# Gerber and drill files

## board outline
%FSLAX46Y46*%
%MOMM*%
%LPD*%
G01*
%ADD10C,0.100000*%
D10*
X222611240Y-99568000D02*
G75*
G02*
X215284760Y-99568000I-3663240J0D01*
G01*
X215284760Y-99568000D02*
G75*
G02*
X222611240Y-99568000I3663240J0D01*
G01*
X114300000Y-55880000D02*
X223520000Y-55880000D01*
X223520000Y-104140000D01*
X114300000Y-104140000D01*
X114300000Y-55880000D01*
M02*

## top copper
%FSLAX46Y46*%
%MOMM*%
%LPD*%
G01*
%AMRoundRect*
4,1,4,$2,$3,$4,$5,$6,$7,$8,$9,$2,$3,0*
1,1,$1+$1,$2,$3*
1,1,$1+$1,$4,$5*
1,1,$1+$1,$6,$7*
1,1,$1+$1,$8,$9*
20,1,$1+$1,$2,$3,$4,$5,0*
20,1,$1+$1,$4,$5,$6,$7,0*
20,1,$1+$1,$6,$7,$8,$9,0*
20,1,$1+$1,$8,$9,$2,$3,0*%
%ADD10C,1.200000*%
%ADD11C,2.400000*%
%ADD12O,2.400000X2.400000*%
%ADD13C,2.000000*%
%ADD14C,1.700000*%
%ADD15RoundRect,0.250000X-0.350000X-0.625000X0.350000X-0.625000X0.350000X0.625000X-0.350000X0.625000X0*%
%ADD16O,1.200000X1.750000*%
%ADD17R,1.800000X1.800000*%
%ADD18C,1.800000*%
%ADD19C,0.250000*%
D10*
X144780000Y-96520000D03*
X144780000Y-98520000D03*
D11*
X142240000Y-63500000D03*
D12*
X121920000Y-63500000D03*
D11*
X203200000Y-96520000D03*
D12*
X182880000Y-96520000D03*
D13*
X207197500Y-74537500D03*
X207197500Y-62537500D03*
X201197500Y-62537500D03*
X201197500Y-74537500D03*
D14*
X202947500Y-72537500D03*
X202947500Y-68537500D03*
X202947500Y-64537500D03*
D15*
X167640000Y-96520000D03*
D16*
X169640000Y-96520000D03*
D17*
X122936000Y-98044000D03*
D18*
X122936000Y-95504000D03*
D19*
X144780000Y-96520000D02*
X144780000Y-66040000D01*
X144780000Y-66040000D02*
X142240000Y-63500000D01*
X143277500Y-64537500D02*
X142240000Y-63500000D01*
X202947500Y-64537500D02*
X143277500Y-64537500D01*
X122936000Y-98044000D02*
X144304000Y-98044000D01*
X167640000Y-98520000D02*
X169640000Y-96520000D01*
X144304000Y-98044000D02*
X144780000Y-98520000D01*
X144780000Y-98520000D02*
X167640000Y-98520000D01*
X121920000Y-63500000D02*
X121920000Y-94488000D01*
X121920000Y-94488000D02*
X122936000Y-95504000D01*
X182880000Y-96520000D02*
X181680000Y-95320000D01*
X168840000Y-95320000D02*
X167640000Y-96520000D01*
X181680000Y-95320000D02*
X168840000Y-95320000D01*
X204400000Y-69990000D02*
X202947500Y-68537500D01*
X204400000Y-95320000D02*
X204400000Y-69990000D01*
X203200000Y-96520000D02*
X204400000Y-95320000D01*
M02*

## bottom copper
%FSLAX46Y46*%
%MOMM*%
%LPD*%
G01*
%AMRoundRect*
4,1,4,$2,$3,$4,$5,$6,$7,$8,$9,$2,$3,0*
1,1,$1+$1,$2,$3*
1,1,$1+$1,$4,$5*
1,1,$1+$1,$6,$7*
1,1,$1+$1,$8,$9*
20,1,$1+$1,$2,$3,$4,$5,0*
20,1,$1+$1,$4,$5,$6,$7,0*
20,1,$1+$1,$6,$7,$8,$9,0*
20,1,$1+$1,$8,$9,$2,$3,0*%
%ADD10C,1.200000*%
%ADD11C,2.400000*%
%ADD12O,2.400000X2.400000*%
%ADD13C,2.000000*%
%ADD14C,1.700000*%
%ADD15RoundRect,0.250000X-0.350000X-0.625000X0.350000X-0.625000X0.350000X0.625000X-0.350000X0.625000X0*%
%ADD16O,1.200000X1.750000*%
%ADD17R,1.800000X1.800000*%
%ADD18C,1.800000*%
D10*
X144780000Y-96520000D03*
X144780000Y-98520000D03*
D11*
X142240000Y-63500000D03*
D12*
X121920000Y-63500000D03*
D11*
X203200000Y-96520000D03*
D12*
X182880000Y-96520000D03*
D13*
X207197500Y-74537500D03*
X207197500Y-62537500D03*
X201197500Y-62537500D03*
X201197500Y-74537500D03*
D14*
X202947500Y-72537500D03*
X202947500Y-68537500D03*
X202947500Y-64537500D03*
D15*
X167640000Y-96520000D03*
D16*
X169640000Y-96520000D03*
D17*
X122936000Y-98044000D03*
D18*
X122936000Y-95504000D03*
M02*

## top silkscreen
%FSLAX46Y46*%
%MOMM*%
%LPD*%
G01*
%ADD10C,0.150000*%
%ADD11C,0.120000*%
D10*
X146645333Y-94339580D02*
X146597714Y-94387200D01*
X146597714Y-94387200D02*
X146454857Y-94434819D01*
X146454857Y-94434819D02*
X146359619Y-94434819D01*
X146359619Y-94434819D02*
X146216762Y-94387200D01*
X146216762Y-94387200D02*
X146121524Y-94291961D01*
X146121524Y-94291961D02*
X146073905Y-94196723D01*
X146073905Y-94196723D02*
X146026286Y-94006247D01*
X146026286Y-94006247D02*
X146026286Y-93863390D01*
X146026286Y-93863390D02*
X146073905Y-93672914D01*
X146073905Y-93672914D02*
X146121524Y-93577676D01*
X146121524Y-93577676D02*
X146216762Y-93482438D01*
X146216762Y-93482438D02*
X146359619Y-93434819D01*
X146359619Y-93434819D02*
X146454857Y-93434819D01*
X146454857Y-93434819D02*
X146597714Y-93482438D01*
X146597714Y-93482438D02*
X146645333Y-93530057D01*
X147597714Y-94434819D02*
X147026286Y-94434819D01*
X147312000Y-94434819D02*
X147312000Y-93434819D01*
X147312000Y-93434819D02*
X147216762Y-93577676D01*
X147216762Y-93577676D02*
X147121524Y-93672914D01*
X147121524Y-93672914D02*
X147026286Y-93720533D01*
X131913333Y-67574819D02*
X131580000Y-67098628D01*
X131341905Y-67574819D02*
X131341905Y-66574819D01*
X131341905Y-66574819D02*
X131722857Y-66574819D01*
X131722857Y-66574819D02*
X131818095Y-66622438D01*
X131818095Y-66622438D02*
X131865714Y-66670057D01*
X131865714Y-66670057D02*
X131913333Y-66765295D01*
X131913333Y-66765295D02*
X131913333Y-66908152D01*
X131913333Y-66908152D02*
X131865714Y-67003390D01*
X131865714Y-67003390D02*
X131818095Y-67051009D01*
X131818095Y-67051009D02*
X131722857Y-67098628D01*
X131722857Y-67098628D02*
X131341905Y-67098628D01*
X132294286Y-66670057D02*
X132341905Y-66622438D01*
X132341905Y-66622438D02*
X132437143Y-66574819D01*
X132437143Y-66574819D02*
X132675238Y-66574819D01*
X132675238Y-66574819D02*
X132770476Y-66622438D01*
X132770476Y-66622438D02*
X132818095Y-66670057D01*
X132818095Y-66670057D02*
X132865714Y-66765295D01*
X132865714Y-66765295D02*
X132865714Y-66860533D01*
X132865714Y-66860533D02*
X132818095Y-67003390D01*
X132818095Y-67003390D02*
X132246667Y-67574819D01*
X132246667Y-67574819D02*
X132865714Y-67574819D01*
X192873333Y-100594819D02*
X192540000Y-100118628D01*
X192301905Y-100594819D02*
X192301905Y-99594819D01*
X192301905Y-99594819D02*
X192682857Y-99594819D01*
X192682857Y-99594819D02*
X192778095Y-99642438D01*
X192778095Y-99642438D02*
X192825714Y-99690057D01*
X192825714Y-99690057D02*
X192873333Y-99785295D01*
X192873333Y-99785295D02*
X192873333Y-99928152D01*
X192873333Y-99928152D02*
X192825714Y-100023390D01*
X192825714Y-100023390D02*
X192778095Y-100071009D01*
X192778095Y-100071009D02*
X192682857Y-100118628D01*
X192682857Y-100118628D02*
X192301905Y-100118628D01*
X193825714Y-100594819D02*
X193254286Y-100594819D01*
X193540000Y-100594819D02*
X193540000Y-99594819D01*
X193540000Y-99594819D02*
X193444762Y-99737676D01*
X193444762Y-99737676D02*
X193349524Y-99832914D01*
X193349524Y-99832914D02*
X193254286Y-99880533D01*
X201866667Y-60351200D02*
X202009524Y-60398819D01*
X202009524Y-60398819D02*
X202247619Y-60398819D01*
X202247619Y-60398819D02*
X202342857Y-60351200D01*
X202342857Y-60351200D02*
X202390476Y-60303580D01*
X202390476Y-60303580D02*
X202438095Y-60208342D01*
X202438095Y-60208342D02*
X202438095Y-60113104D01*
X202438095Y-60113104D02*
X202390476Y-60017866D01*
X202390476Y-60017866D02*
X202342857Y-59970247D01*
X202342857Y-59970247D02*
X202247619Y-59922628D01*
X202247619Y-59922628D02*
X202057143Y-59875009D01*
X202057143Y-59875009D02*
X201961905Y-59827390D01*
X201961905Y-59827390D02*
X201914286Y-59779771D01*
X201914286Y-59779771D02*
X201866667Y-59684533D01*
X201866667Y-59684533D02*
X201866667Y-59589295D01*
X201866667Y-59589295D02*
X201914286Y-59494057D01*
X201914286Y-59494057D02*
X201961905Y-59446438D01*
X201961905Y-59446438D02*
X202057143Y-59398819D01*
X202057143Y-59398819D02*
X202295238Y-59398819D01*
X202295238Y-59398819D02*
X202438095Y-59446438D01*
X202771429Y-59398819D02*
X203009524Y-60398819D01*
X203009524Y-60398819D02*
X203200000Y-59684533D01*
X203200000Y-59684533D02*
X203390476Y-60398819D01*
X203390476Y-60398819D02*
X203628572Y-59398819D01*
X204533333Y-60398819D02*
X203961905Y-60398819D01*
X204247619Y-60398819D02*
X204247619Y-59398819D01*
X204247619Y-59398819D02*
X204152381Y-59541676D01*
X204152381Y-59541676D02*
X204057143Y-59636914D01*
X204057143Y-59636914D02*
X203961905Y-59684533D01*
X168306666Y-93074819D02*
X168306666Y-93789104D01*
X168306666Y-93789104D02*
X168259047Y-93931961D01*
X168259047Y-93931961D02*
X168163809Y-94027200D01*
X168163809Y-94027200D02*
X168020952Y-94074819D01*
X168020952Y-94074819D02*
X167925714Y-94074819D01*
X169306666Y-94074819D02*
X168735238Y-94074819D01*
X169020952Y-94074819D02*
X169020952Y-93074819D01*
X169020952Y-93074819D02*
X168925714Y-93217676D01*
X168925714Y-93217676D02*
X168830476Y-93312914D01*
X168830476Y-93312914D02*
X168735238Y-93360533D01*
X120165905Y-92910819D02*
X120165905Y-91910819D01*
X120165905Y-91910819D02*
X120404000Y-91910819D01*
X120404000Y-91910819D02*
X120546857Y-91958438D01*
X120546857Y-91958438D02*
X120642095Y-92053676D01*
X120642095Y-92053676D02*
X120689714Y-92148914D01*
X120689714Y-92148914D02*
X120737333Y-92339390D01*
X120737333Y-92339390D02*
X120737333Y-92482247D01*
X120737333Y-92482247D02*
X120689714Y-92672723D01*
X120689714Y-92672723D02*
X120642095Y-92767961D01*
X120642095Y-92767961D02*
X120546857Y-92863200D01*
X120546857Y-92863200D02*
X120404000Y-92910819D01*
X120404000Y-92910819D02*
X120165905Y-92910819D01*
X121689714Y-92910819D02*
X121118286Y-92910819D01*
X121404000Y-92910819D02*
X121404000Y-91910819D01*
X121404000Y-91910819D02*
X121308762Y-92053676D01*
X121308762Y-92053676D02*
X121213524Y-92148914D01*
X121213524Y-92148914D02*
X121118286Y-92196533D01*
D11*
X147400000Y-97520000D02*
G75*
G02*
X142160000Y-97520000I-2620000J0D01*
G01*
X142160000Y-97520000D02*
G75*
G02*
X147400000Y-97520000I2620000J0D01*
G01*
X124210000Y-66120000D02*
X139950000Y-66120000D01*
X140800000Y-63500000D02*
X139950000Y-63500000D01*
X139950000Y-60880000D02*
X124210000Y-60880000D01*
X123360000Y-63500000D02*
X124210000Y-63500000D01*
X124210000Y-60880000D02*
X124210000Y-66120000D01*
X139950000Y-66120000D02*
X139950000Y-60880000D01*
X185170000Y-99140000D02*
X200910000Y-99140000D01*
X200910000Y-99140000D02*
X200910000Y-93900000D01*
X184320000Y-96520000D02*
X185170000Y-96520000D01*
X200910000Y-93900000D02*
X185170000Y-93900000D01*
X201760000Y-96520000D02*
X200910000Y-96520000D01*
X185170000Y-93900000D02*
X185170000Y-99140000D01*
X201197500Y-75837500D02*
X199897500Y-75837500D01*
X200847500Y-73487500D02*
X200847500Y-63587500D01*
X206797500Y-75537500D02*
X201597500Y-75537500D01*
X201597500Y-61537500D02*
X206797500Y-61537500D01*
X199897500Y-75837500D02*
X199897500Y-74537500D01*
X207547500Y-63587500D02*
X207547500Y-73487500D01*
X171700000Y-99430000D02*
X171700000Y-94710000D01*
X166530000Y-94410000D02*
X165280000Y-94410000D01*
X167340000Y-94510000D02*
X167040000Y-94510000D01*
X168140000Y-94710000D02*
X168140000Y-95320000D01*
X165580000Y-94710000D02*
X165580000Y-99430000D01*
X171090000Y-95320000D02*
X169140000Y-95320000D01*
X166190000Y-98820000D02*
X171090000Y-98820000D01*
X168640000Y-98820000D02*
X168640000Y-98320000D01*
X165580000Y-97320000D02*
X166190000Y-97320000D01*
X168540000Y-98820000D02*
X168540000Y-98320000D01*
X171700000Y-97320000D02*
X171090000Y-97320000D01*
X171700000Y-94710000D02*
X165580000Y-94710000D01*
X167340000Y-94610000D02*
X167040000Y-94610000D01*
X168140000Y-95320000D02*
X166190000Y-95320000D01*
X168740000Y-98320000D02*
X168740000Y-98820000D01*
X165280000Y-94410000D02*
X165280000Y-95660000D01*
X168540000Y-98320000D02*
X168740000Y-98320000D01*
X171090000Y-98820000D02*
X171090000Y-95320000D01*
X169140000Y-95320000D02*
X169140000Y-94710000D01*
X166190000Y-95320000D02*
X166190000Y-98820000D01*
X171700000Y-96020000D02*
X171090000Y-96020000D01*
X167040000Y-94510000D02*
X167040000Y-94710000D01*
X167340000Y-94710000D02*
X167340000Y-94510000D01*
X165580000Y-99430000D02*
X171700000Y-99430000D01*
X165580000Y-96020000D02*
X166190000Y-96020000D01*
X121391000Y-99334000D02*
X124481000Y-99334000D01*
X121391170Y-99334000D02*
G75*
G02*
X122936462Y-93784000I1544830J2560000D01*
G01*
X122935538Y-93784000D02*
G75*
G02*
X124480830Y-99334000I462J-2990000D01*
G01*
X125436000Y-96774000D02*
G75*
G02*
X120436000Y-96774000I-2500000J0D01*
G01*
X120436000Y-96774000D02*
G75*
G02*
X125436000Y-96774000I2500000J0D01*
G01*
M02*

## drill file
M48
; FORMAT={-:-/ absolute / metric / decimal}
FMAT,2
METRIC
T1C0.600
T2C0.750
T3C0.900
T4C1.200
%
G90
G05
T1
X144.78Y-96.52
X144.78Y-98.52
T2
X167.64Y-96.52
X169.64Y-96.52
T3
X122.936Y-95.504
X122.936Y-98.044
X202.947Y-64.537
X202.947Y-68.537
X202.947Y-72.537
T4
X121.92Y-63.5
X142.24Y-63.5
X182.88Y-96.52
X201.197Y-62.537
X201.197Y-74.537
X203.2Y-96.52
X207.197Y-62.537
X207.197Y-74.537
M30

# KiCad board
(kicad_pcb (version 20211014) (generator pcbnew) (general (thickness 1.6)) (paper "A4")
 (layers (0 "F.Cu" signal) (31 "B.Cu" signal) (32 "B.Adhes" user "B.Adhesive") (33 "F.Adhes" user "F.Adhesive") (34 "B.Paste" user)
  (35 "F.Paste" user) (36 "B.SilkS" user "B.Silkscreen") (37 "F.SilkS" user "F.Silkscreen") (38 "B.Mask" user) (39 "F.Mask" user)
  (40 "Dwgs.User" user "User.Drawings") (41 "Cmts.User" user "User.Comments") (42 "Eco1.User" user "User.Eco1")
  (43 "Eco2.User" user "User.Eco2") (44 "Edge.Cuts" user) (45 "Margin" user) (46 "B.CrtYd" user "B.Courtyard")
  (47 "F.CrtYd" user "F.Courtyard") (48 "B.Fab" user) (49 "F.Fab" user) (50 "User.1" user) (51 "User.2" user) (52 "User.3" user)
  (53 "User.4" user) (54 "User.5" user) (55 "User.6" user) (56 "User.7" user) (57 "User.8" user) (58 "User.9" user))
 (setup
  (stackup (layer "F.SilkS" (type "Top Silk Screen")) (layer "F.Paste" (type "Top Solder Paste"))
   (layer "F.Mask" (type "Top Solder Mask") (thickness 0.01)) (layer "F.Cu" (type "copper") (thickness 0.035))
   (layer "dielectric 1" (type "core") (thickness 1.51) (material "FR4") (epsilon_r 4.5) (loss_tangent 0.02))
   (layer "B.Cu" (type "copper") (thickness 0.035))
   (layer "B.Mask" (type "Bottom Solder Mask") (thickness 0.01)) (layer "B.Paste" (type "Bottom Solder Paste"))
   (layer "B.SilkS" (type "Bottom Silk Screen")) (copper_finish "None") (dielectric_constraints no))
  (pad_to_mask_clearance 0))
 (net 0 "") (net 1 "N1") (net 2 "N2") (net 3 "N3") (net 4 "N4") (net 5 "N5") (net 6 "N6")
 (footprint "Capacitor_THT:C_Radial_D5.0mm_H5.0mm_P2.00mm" (layer "F.Cu") (at 144.78 96.52 -90)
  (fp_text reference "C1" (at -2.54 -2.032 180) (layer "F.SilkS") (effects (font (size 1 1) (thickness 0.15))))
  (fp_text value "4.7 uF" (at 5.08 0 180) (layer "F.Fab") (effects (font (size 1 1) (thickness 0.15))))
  (fp_circle (center 1 0) (end 3.62 0) (layer "F.SilkS") (width 0.12) (fill none))
  (pad "1" thru_hole circle (at 0 0 270) (size 1.2 1.2) (drill 0.6) (layers *.Cu *.Mask) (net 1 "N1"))
  (pad "2" thru_hole circle (at 2 0 270) (size 1.2 1.2) (drill 0.6) (layers *.Cu *.Mask) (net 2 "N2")))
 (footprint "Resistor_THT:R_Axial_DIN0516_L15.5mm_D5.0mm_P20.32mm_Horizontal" (layer "F.Cu") (at 142.24 63.5 180)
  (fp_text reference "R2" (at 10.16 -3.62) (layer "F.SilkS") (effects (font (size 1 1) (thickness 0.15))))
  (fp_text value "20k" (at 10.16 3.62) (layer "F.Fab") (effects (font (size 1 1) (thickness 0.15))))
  (fp_line (start 18.03 -2.62) (end 2.29 -2.62) (layer "F.SilkS") (width 0.12))
  (fp_line (start 1.44 0) (end 2.29 0) (layer "F.SilkS") (width 0.12))
  (fp_line (start 2.29 2.62) (end 18.03 2.62) (layer "F.SilkS") (width 0.12))
  (fp_line (start 18.88 0) (end 18.03 0) (layer "F.SilkS") (width 0.12))
  (fp_line (start 18.03 2.62) (end 18.03 -2.62) (layer "F.SilkS") (width 0.12))
  (fp_line (start 2.29 -2.62) (end 2.29 2.62) (layer "F.SilkS") (width 0.12))
  (pad "1" thru_hole circle (at 0 0 180) (size 2.4 2.4) (drill 1.2) (layers *.Cu *.Mask) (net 1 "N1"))
  (pad "2" thru_hole oval (at 20.32 0 180) (size 2.4 2.4) (drill 1.2) (layers *.Cu *.Mask) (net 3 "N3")))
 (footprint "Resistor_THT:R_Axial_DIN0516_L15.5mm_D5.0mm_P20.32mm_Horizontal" (layer "F.Cu") (at 203.2 96.52 180)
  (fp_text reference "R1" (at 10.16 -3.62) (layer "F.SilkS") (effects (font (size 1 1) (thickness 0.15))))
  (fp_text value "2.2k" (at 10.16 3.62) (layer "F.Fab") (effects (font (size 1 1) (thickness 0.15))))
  (fp_line (start 18.03 -2.62) (end 2.29 -2.62) (layer "F.SilkS") (width 0.12))
  (fp_line (start 2.29 -2.62) (end 2.29 2.62) (layer "F.SilkS") (width 0.12))
  (fp_line (start 18.88 0) (end 18.03 0) (layer "F.SilkS") (width 0.12))
  (fp_line (start 2.29 2.62) (end 18.03 2.62) (layer "F.SilkS") (width 0.12))
  (fp_line (start 1.44 0) (end 2.29 0) (layer "F.SilkS") (width 0.12))
  (fp_line (start 18.03 2.62) (end 18.03 -2.62) (layer "F.SilkS") (width 0.12))
  (pad "1" thru_hole circle (at 0 0 180) (size 2.4 2.4) (drill 1.2) (layers *.Cu *.Mask) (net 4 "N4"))
  (pad "2" thru_hole oval (at 20.32 0 180) (size 2.4 2.4) (drill 1.2) (layers *.Cu *.Mask) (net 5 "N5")))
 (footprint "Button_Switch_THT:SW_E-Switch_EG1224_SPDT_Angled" (layer "F.Cu") (at 202.9475 72.5375 90)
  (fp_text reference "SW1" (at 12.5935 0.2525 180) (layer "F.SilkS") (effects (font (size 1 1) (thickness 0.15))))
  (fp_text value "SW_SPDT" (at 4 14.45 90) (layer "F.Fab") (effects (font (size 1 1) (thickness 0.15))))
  (fp_line (start -3.3 -1.75) (end -3.3 -3.05) (layer "F.SilkS") (width 0.12))
  (fp_line (start -0.95 -2.1) (end 8.95 -2.1) (layer "F.SilkS") (width 0.12))
  (fp_line (start -3 3.85) (end -3 -1.35) (layer "F.SilkS") (width 0.12))
  (fp_line (start 11 -1.35) (end 11 3.85) (layer "F.SilkS") (width 0.12))
  (fp_line (start -3.3 -3.05) (end -2 -3.05) (layer "F.SilkS") (width 0.12))
  (fp_line (start 8.95 4.6) (end -0.95 4.6) (layer "F.SilkS") (width 0.12))
  (pad "" thru_hole circle (at -2 4.25 90) (size 2 2) (drill 1.2) (layers *.Cu *.Mask))
  (pad "" thru_hole circle (at 10 4.25 90) (size 2 2) (drill 1.2) (layers *.Cu *.Mask))
  (pad "" thru_hole circle (at 10 -1.75 90) (size 2 2) (drill 1.2) (layers *.Cu *.Mask))
  (pad "" thru_hole circle (at -2 -1.75 90) (size 2 2) (drill 1.2) (layers *.Cu *.Mask))
  (pad "1" thru_hole circle (at 0 0 90) (size 1.7 1.7) (drill 0.9) (layers *.Cu *.Mask) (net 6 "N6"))
  (pad "2" thru_hole circle (at 4 0 90) (size 1.7 1.7) (drill 0.9) (layers *.Cu *.Mask) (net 4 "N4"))
  (pad "3" thru_hole circle (at 8 0 90) (size 1.7 1.7) (drill 0.9) (layers *.Cu *.Mask) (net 1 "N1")))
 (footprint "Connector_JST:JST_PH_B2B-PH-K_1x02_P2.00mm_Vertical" (layer "F.Cu") (at 167.64 96.52)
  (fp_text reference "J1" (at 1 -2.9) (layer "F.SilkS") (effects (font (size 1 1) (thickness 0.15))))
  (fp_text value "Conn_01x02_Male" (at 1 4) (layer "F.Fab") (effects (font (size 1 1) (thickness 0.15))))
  (fp_line (start 4.06 2.91) (end 4.06 -1.81) (layer "F.SilkS") (width 0.12))
  (fp_line (start -1.11 -2.11) (end -2.36 -2.11) (layer "F.SilkS") (width 0.12))
  (fp_line (start -0.3 -2.01) (end -0.6 -2.01) (layer "F.SilkS") (width 0.12))
  (fp_line (start 0.5 -1.81) (end 0.5 -1.2) (layer "F.SilkS") (width 0.12))
  (fp_line (start -2.06 -1.81) (end -2.06 2.91) (layer "F.SilkS") (width 0.12))
  (fp_line (start 3.45 -1.2) (end 1.5 -1.2) (layer "F.SilkS") (width 0.12))
  (fp_line (start -1.45 2.3) (end 3.45 2.3) (layer "F.SilkS") (width 0.12))
  (fp_line (start 1 2.3) (end 1 1.8) (layer "F.SilkS") (width 0.12))
  (fp_line (start -2.06 0.8) (end -1.45 0.8) (layer "F.SilkS") (width 0.12))
  (fp_line (start 0.9 2.3) (end 0.9 1.8) (layer "F.SilkS") (width 0.12))
  (fp_line (start 4.06 0.8) (end 3.45 0.8) (layer "F.SilkS") (width 0.12))
  (fp_line (start 4.06 -1.81) (end -2.06 -1.81) (layer "F.SilkS") (width 0.12))
  (fp_line (start -0.3 -1.91) (end -0.6 -1.91) (layer "F.SilkS") (width 0.12))
  (fp_line (start 0.5 -1.2) (end -1.45 -1.2) (layer "F.SilkS") (width 0.12))
  (fp_line (start 1.1 1.8) (end 1.1 2.3) (layer "F.SilkS") (width 0.12))
  (fp_line (start -2.36 -2.11) (end -2.36 -0.86) (layer "F.SilkS") (width 0.12))
  (fp_line (start 0.9 1.8) (end 1.1 1.8) (layer "F.SilkS") (width 0.12))
  (fp_line (start 3.45 2.3) (end 3.45 -1.2) (layer "F.SilkS") (width 0.12))
  (fp_line (start 1.5 -1.2) (end 1.5 -1.81) (layer "F.SilkS") (width 0.12))
  (fp_line (start -1.45 -1.2) (end -1.45 2.3) (layer "F.SilkS") (width 0.12))
  (fp_line (start 4.06 -0.5) (end 3.45 -0.5) (layer "F.SilkS") (width 0.12))
  (fp_line (start -0.6 -2.01) (end -0.6 -1.81) (layer "F.SilkS") (width 0.12))
  (fp_line (start -0.3 -1.81) (end -0.3 -2.01) (layer "F.SilkS") (width 0.12))
  (fp_line (start -2.06 2.91) (end 4.06 2.91) (layer "F.SilkS") (width 0.12))
  (fp_line (start -2.06 -0.5) (end -1.45 -0.5) (layer "F.SilkS") (width 0.12))
  (pad "1" thru_hole roundrect (at 0 0) (size 1.2 1.75) (drill 0.75) (layers *.Cu *.Mask) (roundrect_rratio 0.208333) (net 5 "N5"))
  (pad "2" thru_hole oval (at 2 0) (size 1.2 1.75) (drill 0.75) (layers *.Cu *.Mask) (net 2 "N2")))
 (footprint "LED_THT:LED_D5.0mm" (layer "F.Cu") (at 122.936 98.044 90)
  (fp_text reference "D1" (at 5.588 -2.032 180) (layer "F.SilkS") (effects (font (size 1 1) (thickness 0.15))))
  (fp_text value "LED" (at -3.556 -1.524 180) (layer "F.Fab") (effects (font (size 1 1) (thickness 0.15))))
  (fp_line (start -1.29 -1.545) (end -1.29 1.545) (layer "F.SilkS") (width 0.12))
  (fp_arc (start -1.29 -1.54483) (mid 2.072002 -2.880433) (end 4.26 0.000462) (layer "F.SilkS") (width 0.12))
  (fp_arc (start 4.26 -0.000462) (mid 2.072002 2.880433) (end -1.29 1.54483) (layer "F.SilkS") (width 0.12))
  (fp_circle (center 1.27 0) (end 3.77 0) (layer "F.SilkS") (width 0.12) (fill none))
  (pad "1" thru_hole rect (at 0 0 90) (size 1.8 1.8) (drill 0.9) (layers *.Cu *.Mask) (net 2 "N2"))
  (pad "2" thru_hole circle (at 2.54 0 90) (size 1.8 1.8) (drill 0.9) (layers *.Cu *.Mask) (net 3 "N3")))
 (gr_circle (center 218.948 99.568) (end 216.916 96.52) (layer "Edge.Cuts") (width 0.1) (fill none))
 (gr_rect (start 114.3 55.88) (end 223.52 104.14) (layer "Edge.Cuts") (width 0.1) (fill none))
 (segment (start 144.78 96.52) (end 144.78 66.04) (width 0.25) (layer "F.Cu") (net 1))
 (segment (start 144.78 66.04) (end 142.24 63.5) (width 0.25) (layer "F.Cu") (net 1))
 (segment (start 143.2775 64.5375) (end 142.24 63.5) (width 0.25) (layer "F.Cu") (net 1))
 (segment (start 202.9475 64.5375) (end 143.2775 64.5375) (width 0.25) (layer "F.Cu") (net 1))
 (segment (start 122.936 98.044) (end 144.304 98.044) (width 0.25) (layer "F.Cu") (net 2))
 (segment (start 167.64 98.52) (end 169.64 96.52) (width 0.25) (layer "F.Cu") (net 2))
 (segment (start 144.304 98.044) (end 144.78 98.52) (width 0.25) (layer "F.Cu") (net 2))
 (segment (start 144.78 98.52) (end 167.64 98.52) (width 0.25) (layer "F.Cu") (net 2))
 (segment (start 121.92 63.5) (end 121.92 94.488) (width 0.25) (layer "F.Cu") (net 3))
 (segment (start 121.92 94.488) (end 122.936 95.504) (width 0.25) (layer "F.Cu") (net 3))
 (segment (start 182.88 96.52) (end 181.68 95.32) (width 0.25) (layer "F.Cu") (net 5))
 (segment (start 168.84 95.32) (end 167.64 96.52) (width 0.25) (layer "F.Cu") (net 5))
 (segment (start 181.68 95.32) (end 168.84 95.32) (width 0.25) (layer "F.Cu") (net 5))
 (segment (start 204.4 69.99) (end 202.9475 68.5375) (width 0.25) (layer "F.Cu") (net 4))
 (segment (start 204.4 95.32) (end 204.4 69.99) (width 0.25) (layer "F.Cu") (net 4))
 (segment (start 203.2 96.52) (end 204.4 95.32) (width 0.25) (layer "F.Cu") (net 4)))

